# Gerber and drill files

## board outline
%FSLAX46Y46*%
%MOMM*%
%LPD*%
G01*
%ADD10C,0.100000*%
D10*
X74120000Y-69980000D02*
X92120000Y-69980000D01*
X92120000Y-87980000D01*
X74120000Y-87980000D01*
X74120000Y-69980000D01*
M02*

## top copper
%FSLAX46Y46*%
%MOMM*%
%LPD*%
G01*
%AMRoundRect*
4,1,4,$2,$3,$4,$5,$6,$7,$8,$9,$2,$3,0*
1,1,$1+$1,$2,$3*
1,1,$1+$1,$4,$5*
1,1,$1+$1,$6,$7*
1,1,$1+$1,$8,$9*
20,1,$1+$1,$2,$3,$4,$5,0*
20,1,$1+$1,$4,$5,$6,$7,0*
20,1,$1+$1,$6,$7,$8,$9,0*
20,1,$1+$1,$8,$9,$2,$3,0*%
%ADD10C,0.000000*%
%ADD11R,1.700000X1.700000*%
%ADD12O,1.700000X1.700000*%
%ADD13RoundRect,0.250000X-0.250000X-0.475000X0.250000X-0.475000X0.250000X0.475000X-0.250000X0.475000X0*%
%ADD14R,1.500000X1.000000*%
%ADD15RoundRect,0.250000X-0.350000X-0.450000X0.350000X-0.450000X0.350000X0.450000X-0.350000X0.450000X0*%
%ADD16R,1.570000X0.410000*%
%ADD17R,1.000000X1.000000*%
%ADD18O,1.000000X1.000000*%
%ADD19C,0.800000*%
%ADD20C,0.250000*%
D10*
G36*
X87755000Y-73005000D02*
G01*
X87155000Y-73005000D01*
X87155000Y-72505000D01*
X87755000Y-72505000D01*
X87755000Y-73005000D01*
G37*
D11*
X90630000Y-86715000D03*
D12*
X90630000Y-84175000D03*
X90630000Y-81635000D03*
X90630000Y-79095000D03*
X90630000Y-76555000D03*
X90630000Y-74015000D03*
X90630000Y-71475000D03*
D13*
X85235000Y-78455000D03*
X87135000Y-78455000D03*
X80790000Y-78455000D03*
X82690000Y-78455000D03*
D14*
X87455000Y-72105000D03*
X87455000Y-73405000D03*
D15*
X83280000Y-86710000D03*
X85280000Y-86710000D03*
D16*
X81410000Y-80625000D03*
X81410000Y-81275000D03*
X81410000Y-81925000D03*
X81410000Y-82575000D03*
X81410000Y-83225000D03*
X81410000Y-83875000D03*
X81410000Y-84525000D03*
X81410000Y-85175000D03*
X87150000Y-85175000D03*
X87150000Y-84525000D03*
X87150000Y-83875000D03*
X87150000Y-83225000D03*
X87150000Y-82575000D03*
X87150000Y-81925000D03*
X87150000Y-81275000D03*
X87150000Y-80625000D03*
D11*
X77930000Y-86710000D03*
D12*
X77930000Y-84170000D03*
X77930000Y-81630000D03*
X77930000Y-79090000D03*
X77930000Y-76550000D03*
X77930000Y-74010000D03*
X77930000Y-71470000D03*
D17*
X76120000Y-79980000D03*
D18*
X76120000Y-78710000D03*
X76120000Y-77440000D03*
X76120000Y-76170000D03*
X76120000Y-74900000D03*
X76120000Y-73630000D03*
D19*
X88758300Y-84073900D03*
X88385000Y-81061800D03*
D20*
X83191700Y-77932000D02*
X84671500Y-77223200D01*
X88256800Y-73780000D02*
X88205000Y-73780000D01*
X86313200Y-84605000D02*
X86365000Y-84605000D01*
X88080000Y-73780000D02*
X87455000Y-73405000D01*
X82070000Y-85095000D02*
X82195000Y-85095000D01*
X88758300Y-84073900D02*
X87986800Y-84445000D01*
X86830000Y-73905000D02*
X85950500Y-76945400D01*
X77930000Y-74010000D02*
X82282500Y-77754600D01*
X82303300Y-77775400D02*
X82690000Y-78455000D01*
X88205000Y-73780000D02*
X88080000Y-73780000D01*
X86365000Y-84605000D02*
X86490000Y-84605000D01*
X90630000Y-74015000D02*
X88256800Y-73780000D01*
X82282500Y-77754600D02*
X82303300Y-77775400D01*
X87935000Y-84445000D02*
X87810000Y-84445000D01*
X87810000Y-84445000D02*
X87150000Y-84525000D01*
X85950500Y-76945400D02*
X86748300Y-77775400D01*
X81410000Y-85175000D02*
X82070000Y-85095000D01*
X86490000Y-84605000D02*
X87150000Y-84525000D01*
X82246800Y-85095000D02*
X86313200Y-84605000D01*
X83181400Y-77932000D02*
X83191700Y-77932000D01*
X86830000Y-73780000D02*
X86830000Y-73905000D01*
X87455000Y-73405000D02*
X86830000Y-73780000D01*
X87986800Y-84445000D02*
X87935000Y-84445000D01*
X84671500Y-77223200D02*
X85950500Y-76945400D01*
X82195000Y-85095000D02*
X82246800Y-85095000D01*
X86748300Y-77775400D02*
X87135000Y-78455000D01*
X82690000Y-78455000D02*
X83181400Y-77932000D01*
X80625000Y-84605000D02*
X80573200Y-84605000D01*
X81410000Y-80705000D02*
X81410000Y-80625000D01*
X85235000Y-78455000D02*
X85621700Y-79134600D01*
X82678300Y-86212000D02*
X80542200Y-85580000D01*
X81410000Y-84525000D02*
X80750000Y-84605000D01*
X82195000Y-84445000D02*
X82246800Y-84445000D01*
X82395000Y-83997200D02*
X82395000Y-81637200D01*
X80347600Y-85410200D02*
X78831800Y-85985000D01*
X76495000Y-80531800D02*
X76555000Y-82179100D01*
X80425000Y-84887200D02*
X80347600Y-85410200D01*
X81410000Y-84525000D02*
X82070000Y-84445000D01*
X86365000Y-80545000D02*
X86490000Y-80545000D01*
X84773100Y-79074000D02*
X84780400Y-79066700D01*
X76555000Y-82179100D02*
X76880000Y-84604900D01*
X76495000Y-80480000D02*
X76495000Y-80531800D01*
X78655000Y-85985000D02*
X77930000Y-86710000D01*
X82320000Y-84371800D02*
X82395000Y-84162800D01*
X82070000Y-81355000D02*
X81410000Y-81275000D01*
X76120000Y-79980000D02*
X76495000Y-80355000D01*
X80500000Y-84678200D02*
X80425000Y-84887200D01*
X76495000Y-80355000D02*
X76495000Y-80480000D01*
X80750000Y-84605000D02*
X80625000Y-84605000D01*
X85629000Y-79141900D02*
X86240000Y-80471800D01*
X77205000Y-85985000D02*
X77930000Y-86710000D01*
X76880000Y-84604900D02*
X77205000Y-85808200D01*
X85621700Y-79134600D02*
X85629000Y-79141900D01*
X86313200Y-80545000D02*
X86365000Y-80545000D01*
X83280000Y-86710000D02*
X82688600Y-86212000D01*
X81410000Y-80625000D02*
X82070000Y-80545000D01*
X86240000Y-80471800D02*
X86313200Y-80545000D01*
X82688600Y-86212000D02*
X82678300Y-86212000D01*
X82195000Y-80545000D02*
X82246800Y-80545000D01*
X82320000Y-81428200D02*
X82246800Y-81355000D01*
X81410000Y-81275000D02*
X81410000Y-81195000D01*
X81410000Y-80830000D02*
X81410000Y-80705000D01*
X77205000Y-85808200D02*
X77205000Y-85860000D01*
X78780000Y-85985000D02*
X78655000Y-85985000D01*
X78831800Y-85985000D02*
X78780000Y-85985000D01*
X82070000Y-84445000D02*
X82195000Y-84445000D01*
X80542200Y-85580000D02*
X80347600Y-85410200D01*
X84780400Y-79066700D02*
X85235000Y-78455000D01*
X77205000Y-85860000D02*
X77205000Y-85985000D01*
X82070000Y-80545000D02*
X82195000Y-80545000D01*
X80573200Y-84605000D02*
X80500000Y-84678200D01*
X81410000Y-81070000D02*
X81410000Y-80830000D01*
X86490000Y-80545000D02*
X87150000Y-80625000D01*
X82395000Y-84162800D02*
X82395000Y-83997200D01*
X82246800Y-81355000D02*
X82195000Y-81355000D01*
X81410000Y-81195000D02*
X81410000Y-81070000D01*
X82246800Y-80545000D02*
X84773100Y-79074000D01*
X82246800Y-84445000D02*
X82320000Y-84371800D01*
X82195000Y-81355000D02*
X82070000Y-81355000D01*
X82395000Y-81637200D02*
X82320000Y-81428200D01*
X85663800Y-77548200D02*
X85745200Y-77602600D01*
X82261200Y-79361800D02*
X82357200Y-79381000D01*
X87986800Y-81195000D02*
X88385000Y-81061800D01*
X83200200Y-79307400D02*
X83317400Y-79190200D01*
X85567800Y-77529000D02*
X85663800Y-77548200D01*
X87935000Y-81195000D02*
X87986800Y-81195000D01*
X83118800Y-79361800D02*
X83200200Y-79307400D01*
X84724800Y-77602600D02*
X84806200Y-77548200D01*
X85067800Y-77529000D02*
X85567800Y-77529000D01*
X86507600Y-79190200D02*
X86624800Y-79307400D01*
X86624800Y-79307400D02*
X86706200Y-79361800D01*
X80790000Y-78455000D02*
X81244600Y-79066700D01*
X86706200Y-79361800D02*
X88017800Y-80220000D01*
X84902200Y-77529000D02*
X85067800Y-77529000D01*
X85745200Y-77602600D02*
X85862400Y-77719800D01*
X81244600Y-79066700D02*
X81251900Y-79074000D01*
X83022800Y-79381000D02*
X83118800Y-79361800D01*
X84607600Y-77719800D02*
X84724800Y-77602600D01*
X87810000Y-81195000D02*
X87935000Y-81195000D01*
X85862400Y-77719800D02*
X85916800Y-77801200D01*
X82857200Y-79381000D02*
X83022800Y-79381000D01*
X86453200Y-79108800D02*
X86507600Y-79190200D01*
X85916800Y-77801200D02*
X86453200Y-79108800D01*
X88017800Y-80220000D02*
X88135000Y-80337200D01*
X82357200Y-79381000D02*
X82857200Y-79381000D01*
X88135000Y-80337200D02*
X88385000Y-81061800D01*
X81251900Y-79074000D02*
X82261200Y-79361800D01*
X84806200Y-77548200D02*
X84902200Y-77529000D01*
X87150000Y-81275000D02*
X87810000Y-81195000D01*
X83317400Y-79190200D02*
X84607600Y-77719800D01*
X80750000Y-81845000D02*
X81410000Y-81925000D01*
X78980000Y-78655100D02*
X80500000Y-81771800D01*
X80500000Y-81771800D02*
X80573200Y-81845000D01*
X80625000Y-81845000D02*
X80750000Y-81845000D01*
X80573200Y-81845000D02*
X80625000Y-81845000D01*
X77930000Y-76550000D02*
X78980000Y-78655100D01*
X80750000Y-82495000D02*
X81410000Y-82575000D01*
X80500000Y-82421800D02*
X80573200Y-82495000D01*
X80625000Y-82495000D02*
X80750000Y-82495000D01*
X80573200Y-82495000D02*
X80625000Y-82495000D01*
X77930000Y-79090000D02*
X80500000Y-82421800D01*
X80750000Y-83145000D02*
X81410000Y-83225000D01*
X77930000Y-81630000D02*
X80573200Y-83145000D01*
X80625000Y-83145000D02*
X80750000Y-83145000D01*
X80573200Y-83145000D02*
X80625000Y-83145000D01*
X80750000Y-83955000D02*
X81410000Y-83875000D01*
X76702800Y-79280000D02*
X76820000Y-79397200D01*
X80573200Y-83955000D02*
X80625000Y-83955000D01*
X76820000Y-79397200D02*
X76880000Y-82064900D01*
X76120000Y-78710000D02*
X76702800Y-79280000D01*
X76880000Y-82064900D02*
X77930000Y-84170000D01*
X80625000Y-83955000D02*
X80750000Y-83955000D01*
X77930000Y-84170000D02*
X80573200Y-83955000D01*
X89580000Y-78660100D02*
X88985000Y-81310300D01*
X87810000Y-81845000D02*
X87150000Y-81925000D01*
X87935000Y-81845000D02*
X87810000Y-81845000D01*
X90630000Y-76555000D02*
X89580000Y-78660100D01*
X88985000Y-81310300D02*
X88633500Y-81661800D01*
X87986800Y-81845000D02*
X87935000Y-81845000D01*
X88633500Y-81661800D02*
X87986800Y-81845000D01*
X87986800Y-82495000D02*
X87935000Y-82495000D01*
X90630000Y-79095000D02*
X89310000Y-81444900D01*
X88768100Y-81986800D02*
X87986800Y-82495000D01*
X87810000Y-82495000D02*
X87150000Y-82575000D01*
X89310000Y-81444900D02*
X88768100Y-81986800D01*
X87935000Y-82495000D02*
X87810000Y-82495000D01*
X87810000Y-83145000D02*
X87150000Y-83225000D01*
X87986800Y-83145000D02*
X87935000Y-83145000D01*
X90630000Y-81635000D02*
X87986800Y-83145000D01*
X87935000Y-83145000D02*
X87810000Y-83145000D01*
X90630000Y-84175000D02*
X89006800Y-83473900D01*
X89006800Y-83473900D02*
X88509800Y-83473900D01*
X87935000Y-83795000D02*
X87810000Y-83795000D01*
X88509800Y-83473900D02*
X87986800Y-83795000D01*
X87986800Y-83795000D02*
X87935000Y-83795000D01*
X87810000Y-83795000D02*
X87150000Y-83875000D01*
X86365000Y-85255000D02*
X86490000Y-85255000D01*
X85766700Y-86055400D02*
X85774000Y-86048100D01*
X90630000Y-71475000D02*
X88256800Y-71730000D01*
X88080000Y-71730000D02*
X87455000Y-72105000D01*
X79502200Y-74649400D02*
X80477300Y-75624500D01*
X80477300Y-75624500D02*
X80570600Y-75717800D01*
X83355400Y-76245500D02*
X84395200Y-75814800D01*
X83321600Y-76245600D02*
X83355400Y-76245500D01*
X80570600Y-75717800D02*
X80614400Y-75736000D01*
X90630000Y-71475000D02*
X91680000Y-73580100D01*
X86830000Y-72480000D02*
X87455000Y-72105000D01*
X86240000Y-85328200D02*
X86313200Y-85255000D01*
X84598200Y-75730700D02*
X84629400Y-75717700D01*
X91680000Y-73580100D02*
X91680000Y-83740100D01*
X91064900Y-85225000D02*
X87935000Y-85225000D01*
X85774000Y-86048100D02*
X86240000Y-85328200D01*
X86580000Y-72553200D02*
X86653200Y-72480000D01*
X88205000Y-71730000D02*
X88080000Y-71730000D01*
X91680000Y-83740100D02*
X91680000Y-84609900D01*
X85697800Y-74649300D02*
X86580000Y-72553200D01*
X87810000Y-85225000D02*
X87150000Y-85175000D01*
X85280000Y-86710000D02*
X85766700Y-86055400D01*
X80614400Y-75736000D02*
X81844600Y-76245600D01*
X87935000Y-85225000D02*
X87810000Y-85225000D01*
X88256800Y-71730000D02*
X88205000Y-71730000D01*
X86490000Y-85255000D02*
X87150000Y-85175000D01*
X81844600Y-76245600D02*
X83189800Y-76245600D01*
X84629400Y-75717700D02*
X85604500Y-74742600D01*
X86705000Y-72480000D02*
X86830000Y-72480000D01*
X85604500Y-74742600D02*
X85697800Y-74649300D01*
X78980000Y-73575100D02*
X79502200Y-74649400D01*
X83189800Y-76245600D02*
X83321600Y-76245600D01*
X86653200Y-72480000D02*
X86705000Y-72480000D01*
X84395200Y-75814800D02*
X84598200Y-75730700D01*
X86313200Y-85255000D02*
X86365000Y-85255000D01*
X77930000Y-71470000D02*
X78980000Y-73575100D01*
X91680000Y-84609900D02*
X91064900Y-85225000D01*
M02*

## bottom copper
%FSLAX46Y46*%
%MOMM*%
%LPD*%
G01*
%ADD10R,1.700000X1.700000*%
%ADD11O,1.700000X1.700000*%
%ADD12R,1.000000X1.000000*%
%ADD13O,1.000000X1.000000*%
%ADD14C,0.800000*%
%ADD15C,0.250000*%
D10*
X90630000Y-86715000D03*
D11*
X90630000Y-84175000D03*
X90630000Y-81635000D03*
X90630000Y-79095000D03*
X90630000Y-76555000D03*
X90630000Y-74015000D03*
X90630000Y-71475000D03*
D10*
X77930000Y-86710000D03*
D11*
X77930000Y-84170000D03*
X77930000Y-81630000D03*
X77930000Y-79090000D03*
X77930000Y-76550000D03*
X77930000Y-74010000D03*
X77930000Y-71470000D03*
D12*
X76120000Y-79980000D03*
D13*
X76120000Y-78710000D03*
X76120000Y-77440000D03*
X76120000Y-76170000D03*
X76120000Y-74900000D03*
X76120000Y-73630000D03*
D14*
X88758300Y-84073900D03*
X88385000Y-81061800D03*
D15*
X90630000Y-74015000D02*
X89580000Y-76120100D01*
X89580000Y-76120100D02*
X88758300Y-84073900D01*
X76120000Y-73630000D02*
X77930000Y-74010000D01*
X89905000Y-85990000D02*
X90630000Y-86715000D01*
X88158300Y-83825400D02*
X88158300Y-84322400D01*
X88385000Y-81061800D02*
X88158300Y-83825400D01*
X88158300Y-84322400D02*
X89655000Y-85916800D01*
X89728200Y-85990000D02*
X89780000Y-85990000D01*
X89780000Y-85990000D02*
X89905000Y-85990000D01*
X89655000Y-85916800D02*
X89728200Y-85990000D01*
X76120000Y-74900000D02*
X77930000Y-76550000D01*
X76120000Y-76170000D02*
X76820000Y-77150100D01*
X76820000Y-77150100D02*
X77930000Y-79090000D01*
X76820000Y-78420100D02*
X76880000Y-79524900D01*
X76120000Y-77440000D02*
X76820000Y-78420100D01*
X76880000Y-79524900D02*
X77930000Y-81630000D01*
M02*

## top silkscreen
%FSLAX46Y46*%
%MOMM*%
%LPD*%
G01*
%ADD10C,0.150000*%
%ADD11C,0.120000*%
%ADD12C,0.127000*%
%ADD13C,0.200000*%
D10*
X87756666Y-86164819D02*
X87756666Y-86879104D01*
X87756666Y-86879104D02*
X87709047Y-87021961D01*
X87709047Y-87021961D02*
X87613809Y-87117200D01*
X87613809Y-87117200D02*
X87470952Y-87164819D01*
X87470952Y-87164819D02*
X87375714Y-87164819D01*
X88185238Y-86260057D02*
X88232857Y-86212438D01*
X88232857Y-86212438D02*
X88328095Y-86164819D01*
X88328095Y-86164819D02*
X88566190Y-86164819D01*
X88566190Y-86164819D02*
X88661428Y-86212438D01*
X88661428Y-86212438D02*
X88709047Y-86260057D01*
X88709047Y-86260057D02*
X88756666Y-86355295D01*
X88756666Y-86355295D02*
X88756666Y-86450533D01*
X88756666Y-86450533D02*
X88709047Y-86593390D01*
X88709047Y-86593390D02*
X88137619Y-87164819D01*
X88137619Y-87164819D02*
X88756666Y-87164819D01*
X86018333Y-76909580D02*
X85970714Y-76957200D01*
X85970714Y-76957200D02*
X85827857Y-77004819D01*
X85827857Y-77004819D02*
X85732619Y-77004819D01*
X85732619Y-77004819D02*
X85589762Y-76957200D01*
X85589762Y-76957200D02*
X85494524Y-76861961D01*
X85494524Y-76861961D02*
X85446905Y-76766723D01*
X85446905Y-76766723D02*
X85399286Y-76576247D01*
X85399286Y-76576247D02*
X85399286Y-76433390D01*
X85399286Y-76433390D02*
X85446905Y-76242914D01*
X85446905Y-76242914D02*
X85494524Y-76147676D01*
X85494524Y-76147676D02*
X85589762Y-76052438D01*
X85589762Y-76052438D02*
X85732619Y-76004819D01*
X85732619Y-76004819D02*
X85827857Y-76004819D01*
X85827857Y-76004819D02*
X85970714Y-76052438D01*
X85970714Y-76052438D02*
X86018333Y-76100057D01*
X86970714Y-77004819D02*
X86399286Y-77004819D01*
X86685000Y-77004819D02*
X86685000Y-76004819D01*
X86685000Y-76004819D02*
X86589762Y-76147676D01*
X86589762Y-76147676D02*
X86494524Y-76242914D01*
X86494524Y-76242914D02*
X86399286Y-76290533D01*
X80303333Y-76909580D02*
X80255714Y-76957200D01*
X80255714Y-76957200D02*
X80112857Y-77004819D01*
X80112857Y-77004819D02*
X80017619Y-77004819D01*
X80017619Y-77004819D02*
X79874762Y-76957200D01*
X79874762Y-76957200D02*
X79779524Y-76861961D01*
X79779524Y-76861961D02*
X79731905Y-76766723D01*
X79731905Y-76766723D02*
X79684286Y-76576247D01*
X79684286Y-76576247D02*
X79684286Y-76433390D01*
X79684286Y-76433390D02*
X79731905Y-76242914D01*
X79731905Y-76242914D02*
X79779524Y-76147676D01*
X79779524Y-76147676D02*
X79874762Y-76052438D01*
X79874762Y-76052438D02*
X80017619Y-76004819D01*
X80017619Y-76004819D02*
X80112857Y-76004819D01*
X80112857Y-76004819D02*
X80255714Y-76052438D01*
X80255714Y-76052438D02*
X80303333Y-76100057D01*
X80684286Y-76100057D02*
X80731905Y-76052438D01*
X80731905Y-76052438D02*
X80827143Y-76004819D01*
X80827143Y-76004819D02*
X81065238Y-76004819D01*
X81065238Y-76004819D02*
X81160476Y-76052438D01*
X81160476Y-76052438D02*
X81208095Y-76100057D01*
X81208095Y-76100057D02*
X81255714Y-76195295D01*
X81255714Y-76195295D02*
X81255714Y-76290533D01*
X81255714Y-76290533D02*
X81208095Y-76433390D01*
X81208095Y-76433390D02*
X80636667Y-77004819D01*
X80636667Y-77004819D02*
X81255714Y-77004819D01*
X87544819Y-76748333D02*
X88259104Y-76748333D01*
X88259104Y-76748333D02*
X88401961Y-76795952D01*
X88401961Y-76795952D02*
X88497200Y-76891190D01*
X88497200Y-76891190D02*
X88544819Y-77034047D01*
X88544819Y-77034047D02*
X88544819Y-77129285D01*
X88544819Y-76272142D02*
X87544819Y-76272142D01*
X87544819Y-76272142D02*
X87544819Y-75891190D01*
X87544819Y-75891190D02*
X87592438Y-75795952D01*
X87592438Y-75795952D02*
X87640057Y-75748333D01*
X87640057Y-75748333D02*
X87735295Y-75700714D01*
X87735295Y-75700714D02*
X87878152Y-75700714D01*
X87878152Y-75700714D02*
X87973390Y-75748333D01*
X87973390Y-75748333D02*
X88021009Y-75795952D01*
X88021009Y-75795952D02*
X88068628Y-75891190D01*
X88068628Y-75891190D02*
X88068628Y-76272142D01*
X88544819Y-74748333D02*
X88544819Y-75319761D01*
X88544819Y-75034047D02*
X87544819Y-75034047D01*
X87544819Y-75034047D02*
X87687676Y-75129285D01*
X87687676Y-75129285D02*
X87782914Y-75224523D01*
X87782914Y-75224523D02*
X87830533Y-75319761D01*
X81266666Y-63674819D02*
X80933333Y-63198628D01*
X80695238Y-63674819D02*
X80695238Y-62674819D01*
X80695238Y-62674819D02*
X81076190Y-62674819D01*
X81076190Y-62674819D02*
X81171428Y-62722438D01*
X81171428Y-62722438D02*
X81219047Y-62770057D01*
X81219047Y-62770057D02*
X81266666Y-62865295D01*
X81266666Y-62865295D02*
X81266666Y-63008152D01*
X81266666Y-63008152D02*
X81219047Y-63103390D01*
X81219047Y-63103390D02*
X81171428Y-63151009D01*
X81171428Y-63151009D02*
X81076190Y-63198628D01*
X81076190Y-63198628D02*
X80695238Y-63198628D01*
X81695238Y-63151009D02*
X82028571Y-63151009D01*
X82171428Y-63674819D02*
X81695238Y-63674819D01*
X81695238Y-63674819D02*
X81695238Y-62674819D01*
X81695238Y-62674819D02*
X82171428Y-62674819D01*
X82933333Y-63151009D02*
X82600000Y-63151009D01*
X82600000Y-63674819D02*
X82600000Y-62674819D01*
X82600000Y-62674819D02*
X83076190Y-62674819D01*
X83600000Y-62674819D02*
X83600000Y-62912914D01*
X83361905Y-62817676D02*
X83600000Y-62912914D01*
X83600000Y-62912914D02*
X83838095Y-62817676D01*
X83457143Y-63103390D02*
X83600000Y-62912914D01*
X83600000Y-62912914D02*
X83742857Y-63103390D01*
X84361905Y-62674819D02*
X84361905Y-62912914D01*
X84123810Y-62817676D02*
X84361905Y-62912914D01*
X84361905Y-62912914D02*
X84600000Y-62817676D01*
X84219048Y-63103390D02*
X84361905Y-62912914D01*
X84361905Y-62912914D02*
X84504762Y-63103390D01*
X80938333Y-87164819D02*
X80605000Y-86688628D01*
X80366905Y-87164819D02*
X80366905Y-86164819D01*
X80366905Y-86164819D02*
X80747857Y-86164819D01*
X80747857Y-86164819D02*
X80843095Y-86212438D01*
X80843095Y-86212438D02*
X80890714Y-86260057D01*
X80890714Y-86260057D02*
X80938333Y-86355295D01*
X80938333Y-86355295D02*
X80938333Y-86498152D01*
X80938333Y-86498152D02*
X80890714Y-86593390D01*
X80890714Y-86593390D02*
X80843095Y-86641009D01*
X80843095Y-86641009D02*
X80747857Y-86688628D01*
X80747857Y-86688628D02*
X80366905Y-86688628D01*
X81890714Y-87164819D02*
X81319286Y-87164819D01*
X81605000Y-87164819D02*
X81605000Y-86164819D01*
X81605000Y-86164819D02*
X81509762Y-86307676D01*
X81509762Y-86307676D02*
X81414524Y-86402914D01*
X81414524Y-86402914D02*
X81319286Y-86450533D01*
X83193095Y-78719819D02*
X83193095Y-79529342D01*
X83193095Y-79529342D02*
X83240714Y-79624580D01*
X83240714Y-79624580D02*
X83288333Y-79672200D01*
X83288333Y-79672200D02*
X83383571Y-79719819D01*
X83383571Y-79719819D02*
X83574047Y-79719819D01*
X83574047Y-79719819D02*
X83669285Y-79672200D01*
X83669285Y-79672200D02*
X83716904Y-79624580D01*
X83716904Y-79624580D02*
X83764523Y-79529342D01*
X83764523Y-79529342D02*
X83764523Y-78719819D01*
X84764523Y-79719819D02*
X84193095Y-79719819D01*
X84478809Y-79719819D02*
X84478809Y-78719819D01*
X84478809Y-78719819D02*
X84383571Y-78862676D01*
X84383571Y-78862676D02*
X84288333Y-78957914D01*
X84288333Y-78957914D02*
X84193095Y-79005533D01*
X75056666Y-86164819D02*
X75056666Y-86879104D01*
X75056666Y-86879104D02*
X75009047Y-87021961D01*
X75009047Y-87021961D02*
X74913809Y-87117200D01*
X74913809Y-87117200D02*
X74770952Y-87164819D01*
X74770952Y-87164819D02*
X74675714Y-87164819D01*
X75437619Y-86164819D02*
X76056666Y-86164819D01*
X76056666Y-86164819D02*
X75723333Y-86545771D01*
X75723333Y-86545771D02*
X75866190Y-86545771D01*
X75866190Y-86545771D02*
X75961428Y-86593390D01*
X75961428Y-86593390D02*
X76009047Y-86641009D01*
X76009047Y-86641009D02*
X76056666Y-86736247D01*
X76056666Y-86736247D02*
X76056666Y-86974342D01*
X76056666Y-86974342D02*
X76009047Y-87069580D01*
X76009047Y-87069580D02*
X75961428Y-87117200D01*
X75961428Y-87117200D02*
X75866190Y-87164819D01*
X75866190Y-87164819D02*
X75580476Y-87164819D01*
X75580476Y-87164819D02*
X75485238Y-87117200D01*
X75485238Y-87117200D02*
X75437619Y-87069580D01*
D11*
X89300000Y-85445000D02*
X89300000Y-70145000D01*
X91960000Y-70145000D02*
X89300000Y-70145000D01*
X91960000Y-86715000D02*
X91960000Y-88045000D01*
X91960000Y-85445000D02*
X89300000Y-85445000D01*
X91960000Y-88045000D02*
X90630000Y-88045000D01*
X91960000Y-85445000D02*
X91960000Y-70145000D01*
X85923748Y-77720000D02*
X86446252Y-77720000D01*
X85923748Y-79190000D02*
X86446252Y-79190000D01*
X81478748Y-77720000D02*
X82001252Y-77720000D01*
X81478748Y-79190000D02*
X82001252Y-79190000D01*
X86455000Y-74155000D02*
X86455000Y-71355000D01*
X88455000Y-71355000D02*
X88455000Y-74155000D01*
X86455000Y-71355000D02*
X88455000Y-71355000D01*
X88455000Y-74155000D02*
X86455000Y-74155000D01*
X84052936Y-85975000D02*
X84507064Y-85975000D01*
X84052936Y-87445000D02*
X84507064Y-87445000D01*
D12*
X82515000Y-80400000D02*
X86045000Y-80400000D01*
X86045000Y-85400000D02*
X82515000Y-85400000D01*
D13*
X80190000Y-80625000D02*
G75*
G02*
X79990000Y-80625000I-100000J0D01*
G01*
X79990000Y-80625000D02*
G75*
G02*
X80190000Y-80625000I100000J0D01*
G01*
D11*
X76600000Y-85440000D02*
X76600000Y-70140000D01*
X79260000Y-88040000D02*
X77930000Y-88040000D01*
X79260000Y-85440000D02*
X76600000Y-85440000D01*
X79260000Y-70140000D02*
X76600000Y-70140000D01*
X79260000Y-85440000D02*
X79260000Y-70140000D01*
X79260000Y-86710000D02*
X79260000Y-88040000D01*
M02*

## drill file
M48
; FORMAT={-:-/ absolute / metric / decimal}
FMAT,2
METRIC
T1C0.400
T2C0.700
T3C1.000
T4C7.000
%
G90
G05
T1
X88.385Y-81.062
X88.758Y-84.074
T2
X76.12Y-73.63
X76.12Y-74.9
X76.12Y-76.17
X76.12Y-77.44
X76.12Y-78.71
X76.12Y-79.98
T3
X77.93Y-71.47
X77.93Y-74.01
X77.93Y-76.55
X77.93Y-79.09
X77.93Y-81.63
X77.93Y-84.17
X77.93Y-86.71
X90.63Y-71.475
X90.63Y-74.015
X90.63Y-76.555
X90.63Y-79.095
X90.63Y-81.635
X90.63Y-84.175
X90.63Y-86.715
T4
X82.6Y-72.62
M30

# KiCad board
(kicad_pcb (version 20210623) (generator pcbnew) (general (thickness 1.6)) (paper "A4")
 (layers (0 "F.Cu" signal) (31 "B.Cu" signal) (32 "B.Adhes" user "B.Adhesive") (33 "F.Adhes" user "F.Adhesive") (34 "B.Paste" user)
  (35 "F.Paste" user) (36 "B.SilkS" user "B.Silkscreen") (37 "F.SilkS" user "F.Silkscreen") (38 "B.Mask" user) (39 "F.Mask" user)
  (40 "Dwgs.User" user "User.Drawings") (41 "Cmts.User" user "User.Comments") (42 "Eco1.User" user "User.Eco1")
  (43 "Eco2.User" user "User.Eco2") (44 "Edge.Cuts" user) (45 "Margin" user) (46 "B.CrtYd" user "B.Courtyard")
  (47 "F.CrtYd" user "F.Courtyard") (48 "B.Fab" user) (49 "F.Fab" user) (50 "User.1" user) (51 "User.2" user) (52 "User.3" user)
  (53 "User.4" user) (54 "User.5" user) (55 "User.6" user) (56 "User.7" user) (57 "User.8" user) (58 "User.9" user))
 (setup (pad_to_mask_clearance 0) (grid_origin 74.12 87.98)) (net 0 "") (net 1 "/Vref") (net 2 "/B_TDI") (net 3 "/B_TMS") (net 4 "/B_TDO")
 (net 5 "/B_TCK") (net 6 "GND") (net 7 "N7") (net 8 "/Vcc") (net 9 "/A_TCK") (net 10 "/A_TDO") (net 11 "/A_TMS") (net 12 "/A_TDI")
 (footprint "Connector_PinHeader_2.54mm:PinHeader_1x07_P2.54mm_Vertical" (layer "F.Cu") (at 90.63 86.715 180)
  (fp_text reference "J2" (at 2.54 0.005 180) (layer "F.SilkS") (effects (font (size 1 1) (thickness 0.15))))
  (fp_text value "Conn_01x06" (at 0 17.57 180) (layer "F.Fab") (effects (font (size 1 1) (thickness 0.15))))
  (fp_line (start 1.33 1.27) (end 1.33 16.57) (layer "F.SilkS") (width 0.12))
  (fp_line (start -1.33 16.57) (end 1.33 16.57) (layer "F.SilkS") (width 0.12))
  (fp_line (start -1.33 0) (end -1.33 -1.33) (layer "F.SilkS") (width 0.12))
  (fp_line (start -1.33 1.27) (end 1.33 1.27) (layer "F.SilkS") (width 0.12))
  (fp_line (start -1.33 -1.33) (end 0 -1.33) (layer "F.SilkS") (width 0.12))
  (fp_line (start -1.33 1.27) (end -1.33 16.57) (layer "F.SilkS") (width 0.12))
  (pad "1" thru_hole rect locked (at 0 0 180) (size 1.7 1.7) (drill 1) (layers *.Cu *.Mask) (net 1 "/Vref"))
  (pad "2" thru_hole oval locked (at 0 2.54 180) (size 1.7 1.7) (drill 1) (layers *.Cu *.Mask) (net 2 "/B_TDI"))
  (pad "3" thru_hole oval locked (at 0 5.08 180) (size 1.7 1.7) (drill 1) (layers *.Cu *.Mask) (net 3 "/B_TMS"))
  (pad "4" thru_hole oval locked (at 0 7.62 180) (size 1.7 1.7) (drill 1) (layers *.Cu *.Mask) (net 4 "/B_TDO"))
  (pad "5" thru_hole oval locked (at 0 10.16 180) (size 1.7 1.7) (drill 1) (layers *.Cu *.Mask) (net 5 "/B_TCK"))
  (pad "6" thru_hole oval locked (at 0 12.7 180) (size 1.7 1.7) (drill 1) (layers *.Cu *.Mask) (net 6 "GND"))
  (pad "7" thru_hole oval locked (at 0 15.24 180) (size 1.7 1.7) (drill 1) (layers *.Cu *.Mask) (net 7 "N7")))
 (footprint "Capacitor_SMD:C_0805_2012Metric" (layer "F.Cu") (at 86.185 78.455)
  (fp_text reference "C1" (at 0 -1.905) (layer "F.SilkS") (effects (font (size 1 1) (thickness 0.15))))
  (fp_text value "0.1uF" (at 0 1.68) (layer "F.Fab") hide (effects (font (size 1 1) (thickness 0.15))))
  (fp_line (start -0.261252 -0.735) (end 0.261252 -0.735) (layer "F.SilkS") (width 0.12))
  (fp_line (start -0.261252 0.735) (end 0.261252 0.735) (layer "F.SilkS") (width 0.12))
  (pad "1" smd roundrect locked (at -0.95 0) (size 1 1.45) (layers "F.Cu" "F.Paste" "F.Mask") (roundrect_rratio 0.25) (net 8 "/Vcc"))
  (pad "2" smd roundrect locked (at 0.95 0) (size 1 1.45) (layers "F.Cu" "F.Paste" "F.Mask") (roundrect_rratio 0.25) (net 6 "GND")))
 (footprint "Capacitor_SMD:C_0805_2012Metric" (layer "F.Cu") (at 81.74 78.455)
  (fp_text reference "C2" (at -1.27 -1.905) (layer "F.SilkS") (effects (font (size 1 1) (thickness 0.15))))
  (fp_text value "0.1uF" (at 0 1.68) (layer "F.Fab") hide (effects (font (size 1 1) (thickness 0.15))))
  (fp_line (start -0.261252 -0.735) (end 0.261252 -0.735) (layer "F.SilkS") (width 0.12))
  (fp_line (start -0.261252 0.735) (end 0.261252 0.735) (layer "F.SilkS") (width 0.12))
  (pad "1" smd roundrect locked (at -0.95 0) (size 1 1.45) (layers "F.Cu" "F.Paste" "F.Mask") (roundrect_rratio 0.25) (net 1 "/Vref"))
  (pad "2" smd roundrect locked (at 0.95 0) (size 1 1.45) (layers "F.Cu" "F.Paste" "F.Mask") (roundrect_rratio 0.25) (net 6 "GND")))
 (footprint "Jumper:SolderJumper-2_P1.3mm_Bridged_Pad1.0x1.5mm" (layer "F.Cu") (at 87.455 72.755 -90)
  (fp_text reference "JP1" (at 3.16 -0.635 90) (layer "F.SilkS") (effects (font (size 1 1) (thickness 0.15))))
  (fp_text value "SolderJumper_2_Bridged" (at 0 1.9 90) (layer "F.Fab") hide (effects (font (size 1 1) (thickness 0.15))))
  (fp_poly (pts (xy -0.25 -0.3) (xy 0.25 -0.3) (xy 0.25 0.3) (xy -0.25 0.3)) (layer "F.Cu") (width 0) (fill solid))
  (fp_line (start 1.4 1) (end -1.4 1) (layer "F.SilkS") (width 0.12))
  (fp_line (start -1.4 -1) (end 1.4 -1) (layer "F.SilkS") (width 0.12))
  (fp_line (start -1.4 1) (end -1.4 -1) (layer "F.SilkS") (width 0.12))
  (fp_line (start 1.4 -1) (end 1.4 1) (layer "F.SilkS") (width 0.12))
  (pad "1" smd rect locked (at -0.65 0 270) (size 1 1.5) (layers "F.Cu" "F.Mask") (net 7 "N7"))
  (pad "2" smd rect locked (at 0.65 0 270) (size 1 1.5) (layers "F.Cu" "F.Mask") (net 6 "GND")))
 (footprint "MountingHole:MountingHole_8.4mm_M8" (layer "F.Cu") (at 82.6 72.62)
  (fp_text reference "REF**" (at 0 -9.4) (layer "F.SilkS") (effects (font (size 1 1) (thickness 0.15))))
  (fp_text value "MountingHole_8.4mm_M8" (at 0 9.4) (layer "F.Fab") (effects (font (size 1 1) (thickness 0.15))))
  (pad "" np_thru_hole circle (at 0 0) (size 7 7) (drill 7) (layers F&B.Cu *.Mask)))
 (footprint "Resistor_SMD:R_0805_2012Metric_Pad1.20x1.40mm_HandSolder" (layer "F.Cu") (at 84.28 86.71)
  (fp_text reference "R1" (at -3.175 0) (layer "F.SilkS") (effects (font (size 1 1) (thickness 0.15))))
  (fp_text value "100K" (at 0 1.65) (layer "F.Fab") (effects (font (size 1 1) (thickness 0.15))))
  (fp_line (start -0.227064 -0.735) (end 0.227064 -0.735) (layer "F.SilkS") (width 0.12))
  (fp_line (start -0.227064 0.735) (end 0.227064 0.735) (layer "F.SilkS") (width 0.12))
  (pad "1" smd roundrect locked (at -1 0) (size 1.2 1.4) (layers "F.Cu" "F.Paste" "F.Mask") (roundrect_rratio 0.208333) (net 8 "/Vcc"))
  (pad "2" smd roundrect locked (at 1 0) (size 1.2 1.4) (layers "F.Cu" "F.Paste" "F.Mask") (roundrect_rratio 0.208333) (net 7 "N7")))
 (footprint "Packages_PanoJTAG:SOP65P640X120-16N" (layer "F.Cu") (at 84.28 82.9)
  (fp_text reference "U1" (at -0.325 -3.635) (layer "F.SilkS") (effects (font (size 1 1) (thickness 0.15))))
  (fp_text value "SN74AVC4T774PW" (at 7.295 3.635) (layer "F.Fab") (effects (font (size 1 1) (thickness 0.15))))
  (fp_line (start -1.765 -2.5) (end 1.765 -2.5) (layer "F.SilkS") (width 0.127))
  (fp_line (start 1.765 2.5) (end -1.765 2.5) (layer "F.SilkS") (width 0.127))
  (fp_circle (center -4.19 -2.275) (end -4.09 -2.275) (layer "F.SilkS") (width 0.2) (fill none))
  (pad "1" smd rect locked (at -2.87 -2.275) (size 1.57 0.41) (layers "F.Cu" "F.Paste" "F.Mask") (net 8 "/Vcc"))
  (pad "2" smd rect locked (at -2.87 -1.625) (size 1.57 0.41) (layers "F.Cu" "F.Paste" "F.Mask") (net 8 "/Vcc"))
  (pad "3" smd rect locked (at -2.87 -0.975) (size 1.57 0.41) (layers "F.Cu" "F.Paste" "F.Mask") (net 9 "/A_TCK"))
  (pad "4" smd rect locked (at -2.87 -0.325) (size 1.57 0.41) (layers "F.Cu" "F.Paste" "F.Mask") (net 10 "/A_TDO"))
  (pad "5" smd rect locked (at -2.87 0.325) (size 1.57 0.41) (layers "F.Cu" "F.Paste" "F.Mask") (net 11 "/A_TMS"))
  (pad "6" smd rect locked (at -2.87 0.975) (size 1.57 0.41) (layers "F.Cu" "F.Paste" "F.Mask") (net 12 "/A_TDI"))
  (pad "7" smd rect locked (at -2.87 1.625) (size 1.57 0.41) (layers "F.Cu" "F.Paste" "F.Mask") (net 8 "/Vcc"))
  (pad "8" smd rect locked (at -2.87 2.275) (size 1.57 0.41) (layers "F.Cu" "F.Paste" "F.Mask") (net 6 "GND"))
  (pad "9" smd rect locked (at 2.87 2.275) (size 1.57 0.41) (layers "F.Cu" "F.Paste" "F.Mask") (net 7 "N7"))
  (pad "10" smd rect locked (at 2.87 1.625) (size 1.57 0.41) (layers "F.Cu" "F.Paste" "F.Mask") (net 6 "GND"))
  (pad "11" smd rect locked (at 2.87 0.975) (size 1.57 0.41) (layers "F.Cu" "F.Paste" "F.Mask") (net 2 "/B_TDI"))
  (pad "12" smd rect locked (at 2.87 0.325) (size 1.57 0.41) (layers "F.Cu" "F.Paste" "F.Mask") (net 3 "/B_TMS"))
  (pad "13" smd rect locked (at 2.87 -0.325) (size 1.57 0.41) (layers "F.Cu" "F.Paste" "F.Mask") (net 4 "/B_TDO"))
  (pad "14" smd rect locked (at 2.87 -0.975) (size 1.57 0.41) (layers "F.Cu" "F.Paste" "F.Mask") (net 5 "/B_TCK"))
  (pad "15" smd rect locked (at 2.87 -1.625) (size 1.57 0.41) (layers "F.Cu" "F.Paste" "F.Mask") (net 1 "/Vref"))
  (pad "16" smd rect locked (at 2.87 -2.275) (size 1.57 0.41) (layers "F.Cu" "F.Paste" "F.Mask") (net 8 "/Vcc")))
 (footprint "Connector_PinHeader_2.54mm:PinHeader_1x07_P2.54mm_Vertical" (layer "F.Cu") (at 77.93 86.71 180)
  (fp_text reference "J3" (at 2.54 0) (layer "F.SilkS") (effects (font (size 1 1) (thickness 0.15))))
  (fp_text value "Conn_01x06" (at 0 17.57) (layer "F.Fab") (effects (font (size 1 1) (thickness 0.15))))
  (fp_line (start 1.33 1.27) (end 1.33 16.57) (layer "F.SilkS") (width 0.12))
  (fp_line (start -1.33 -1.33) (end 0 -1.33) (layer "F.SilkS") (width 0.12))
  (fp_line (start -1.33 1.27) (end 1.33 1.27) (layer "F.SilkS") (width 0.12))
  (fp_line (start -1.33 16.57) (end 1.33 16.57) (layer "F.SilkS") (width 0.12))
  (fp_line (start -1.33 1.27) (end -1.33 16.57) (layer "F.SilkS") (width 0.12))
  (fp_line (start -1.33 0) (end -1.33 -1.33) (layer "F.SilkS") (width 0.12))
  (pad "1" thru_hole rect locked (at 0 0 180) (size 1.7 1.7) (drill 1) (layers *.Cu *.Mask) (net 8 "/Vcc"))
  (pad "2" thru_hole oval locked (at 0 2.54 180) (size 1.7 1.7) (drill 1) (layers *.Cu *.Mask) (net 12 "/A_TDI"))
  (pad "3" thru_hole oval locked (at 0 5.08 180) (size 1.7 1.7) (drill 1) (layers *.Cu *.Mask) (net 11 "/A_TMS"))
  (pad "4" thru_hole oval locked (at 0 7.62 180) (size 1.7 1.7) (drill 1) (layers *.Cu *.Mask) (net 10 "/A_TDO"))
  (pad "5" thru_hole oval locked (at 0 10.16 180) (size 1.7 1.7) (drill 1) (layers *.Cu *.Mask) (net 9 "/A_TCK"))
  (pad "6" thru_hole oval locked (at 0 12.7 180) (size 1.7 1.7) (drill 1) (layers *.Cu *.Mask) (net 6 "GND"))
  (pad "7" thru_hole oval locked (at 0 15.24 180) (size 1.7 1.7) (drill 1) (layers *.Cu *.Mask) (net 7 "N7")))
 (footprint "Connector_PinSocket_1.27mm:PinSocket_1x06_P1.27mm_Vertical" (layer "B.Cu") (at 76.12 79.98)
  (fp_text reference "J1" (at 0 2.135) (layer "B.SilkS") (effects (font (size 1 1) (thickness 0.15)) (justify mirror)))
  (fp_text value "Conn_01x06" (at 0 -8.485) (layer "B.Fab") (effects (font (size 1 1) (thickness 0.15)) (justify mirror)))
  (pad "1" thru_hole rect locked (at 0 0) (size 1 1) (drill 0.7) (layers *.Cu *.Mask) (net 8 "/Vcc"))
  (pad "2" thru_hole oval locked (at 0 -1.27) (size 1 1) (drill 0.7) (layers *.Cu *.Mask) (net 12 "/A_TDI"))
  (pad "3" thru_hole oval locked (at 0 -2.54) (size 1 1) (drill 0.7) (layers *.Cu *.Mask) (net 11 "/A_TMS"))
  (pad "4" thru_hole oval locked (at 0 -3.81) (size 1 1) (drill 0.7) (layers *.Cu *.Mask) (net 10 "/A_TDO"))
  (pad "5" thru_hole oval locked (at 0 -5.08) (size 1 1) (drill 0.7) (layers *.Cu *.Mask) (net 9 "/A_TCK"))
  (pad "6" thru_hole oval locked (at 0 -6.35) (size 1 1) (drill 0.7) (layers *.Cu *.Mask) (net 6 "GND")))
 (gr_rect (start 92.12 87.98) (end 74.12 69.98) (layer "Edge.Cuts") (width 0.1) (fill none))
 (segment (start 83.1917 77.932) (end 84.6715 77.2232) (width 0.25) (layer "F.Cu") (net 6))
 (segment (start 88.2568 73.78) (end 88.205 73.78) (width 0.25) (layer "F.Cu") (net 6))
 (segment (start 86.3132 84.605) (end 86.365 84.605) (width 0.25) (layer "F.Cu") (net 6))
 (segment (start 88.08 73.78) (end 87.455 73.405) (width 0.25) (layer "F.Cu") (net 6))
 (segment (start 82.07 85.095) (end 82.195 85.095) (width 0.25) (layer "F.Cu") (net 6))
 (segment (start 88.7583 84.0739) (end 87.9868 84.445) (width 0.25) (layer "F.Cu") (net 6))
 (segment (start 86.83 73.905) (end 85.9505 76.9454) (width 0.25) (layer "F.Cu") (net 6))
 (segment (start 77.93 74.01) (end 82.2825 77.7546) (width 0.25) (layer "F.Cu") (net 6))
 (segment (start 82.3033 77.7754) (end 82.69 78.455) (width 0.25) (layer "F.Cu") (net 6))
 (segment (start 88.205 73.78) (end 88.08 73.78) (width 0.25) (layer "F.Cu") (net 6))
 (segment (start 86.365 84.605) (end 86.49 84.605) (width 0.25) (layer "F.Cu") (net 6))
 (segment (start 90.63 74.015) (end 88.2568 73.78) (width 0.25) (layer "F.Cu") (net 6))
 (segment (start 82.2825 77.7546) (end 82.3033 77.7754) (width 0.25) (layer "F.Cu") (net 6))
 (segment (start 87.935 84.445) (end 87.81 84.445) (width 0.25) (layer "F.Cu") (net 6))
 (segment (start 87.81 84.445) (end 87.15 84.525) (width 0.25) (layer "F.Cu") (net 6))
 (segment (start 85.9505 76.9454) (end 86.7483 77.7754) (width 0.25) (layer "F.Cu") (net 6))
 (segment (start 81.41 85.175) (end 82.07 85.095) (width 0.25) (layer "F.Cu") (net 6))
 (segment (start 86.49 84.605) (end 87.15 84.525) (width 0.25) (layer "F.Cu") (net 6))
 (segment (start 82.2468 85.095) (end 86.3132 84.605) (width 0.25) (layer "F.Cu") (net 6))
 (segment (start 83.1814 77.932) (end 83.1917 77.932) (width 0.25) (layer "F.Cu") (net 6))
 (segment (start 86.83 73.78) (end 86.83 73.905) (width 0.25) (layer "F.Cu") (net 6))
 (segment (start 87.455 73.405) (end 86.83 73.78) (width 0.25) (layer "F.Cu") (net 6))
 (segment (start 87.9868 84.445) (end 87.935 84.445) (width 0.25) (layer "F.Cu") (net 6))
 (segment (start 84.6715 77.2232) (end 85.9505 76.9454) (width 0.25) (layer "F.Cu") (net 6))
 (segment (start 82.195 85.095) (end 82.2468 85.095) (width 0.25) (layer "F.Cu") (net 6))
 (segment (start 86.7483 77.7754) (end 87.135 78.455) (width 0.25) (layer "F.Cu") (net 6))
 (segment (start 82.69 78.455) (end 83.1814 77.932) (width 0.25) (layer "F.Cu") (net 6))
 (via (at 88.7583 84.0739) (size 0.8) (drill 0.4) (layers "F.Cu" "B.Cu") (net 6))
 (segment (start 90.63 74.015) (end 89.58 76.1201) (width 0.25) (layer "B.Cu") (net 6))
 (segment (start 89.58 76.1201) (end 88.7583 84.0739) (width 0.25) (layer "B.Cu") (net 6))
 (segment (start 76.12 73.63) (end 77.93 74.01) (width 0.25) (layer "B.Cu") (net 6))
 (segment (start 80.625 84.605) (end 80.5732 84.605) (width 0.25) (layer "F.Cu") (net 8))
 (segment (start 81.41 80.705) (end 81.41 80.625) (width 0.25) (layer "F.Cu") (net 8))
 (segment (start 85.235 78.455) (end 85.6217 79.1346) (width 0.25) (layer "F.Cu") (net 8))
 (segment (start 82.6783 86.212) (end 80.5422 85.58) (width 0.25) (layer "F.Cu") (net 8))
 (segment (start 81.41 84.525) (end 80.75 84.605) (width 0.25) (layer "F.Cu") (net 8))
 (segment (start 82.195 84.445) (end 82.2468 84.445) (width 0.25) (layer "F.Cu") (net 8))
 (segment (start 82.395 83.9972) (end 82.395 81.6372) (width 0.25) (layer "F.Cu") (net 8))
 (segment (start 80.3476 85.4102) (end 78.8318 85.985) (width 0.25) (layer "F.Cu") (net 8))
 (segment (start 76.495 80.5318) (end 76.555 82.1791) (width 0.25) (layer "F.Cu") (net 8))
 (segment (start 80.425 84.8872) (end 80.3476 85.4102) (width 0.25) (layer "F.Cu") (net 8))
 (segment (start 81.41 84.525) (end 82.07 84.445) (width 0.25) (layer "F.Cu") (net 8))
 (segment (start 86.365 80.545) (end 86.49 80.545) (width 0.25) (layer "F.Cu") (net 8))
 (segment (start 84.7731 79.074) (end 84.7804 79.0667) (width 0.25) (layer "F.Cu") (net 8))
 (segment (start 76.555 82.1791) (end 76.88 84.6049) (width 0.25) (layer "F.Cu") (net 8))
 (segment (start 76.495 80.48) (end 76.495 80.5318) (width 0.25) (layer "F.Cu") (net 8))
 (segment (start 78.655 85.985) (end 77.93 86.71) (width 0.25) (layer "F.Cu") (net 8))
 (segment (start 82.32 84.3718) (end 82.395 84.1628) (width 0.25) (layer "F.Cu") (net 8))
 (segment (start 82.07 81.355) (end 81.41 81.275) (width 0.25) (layer "F.Cu") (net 8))
 (segment (start 76.12 79.98) (end 76.495 80.355) (width 0.25) (layer "F.Cu") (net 8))
 (segment (start 80.5 84.6782) (end 80.425 84.8872) (width 0.25) (layer "F.Cu") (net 8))
 (segment (start 76.495 80.355) (end 76.495 80.48) (width 0.25) (layer "F.Cu") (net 8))
 (segment (start 80.75 84.605) (end 80.625 84.605) (width 0.25) (layer "F.Cu") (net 8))
 (segment (start 85.629 79.1419) (end 86.24 80.4718) (width 0.25) (layer "F.Cu") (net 8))
 (segment (start 77.205 85.985) (end 77.93 86.71) (width 0.25) (layer "F.Cu") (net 8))
 (segment (start 76.88 84.6049) (end 77.205 85.8082) (width 0.25) (layer "F.Cu") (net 8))
 (segment (start 85.6217 79.1346) (end 85.629 79.1419) (width 0.25) (layer "F.Cu") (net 8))
 (segment (start 86.3132 80.545) (end 86.365 80.545) (width 0.25) (layer "F.Cu") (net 8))
 (segment (start 83.28 86.71) (end 82.6886 86.212) (width 0.25) (layer "F.Cu") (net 8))
 (segment (start 81.41 80.625) (end 82.07 80.545) (width 0.25) (layer "F.Cu") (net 8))
 (segment (start 86.24 80.4718) (end 86.3132 80.545) (width 0.25) (layer "F.Cu") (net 8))
 (segment (start 82.6886 86.212) (end 82.6783 86.212) (width 0.25) (layer "F.Cu") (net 8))
 (segment (start 82.195 80.545) (end 82.2468 80.545) (width 0.25) (layer "F.Cu") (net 8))
 (segment (start 82.32 81.4282) (end 82.2468 81.355) (width 0.25) (layer "F.Cu") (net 8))
 (segment (start 81.41 81.275) (end 81.41 81.195) (width 0.25) (layer "F.Cu") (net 8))
 (segment (start 81.41 80.83) (end 81.41 80.705) (width 0.25) (layer "F.Cu") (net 8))
 (segment (start 77.205 85.8082) (end 77.205 85.86) (width 0.25) (layer "F.Cu") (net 8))
 (segment (start 78.78 85.985) (end 78.655 85.985) (width 0.25) (layer "F.Cu") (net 8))
 (segment (start 78.8318 85.985) (end 78.78 85.985) (width 0.25) (layer "F.Cu") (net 8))
 (segment (start 82.07 84.445) (end 82.195 84.445) (width 0.25) (layer "F.Cu") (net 8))
 (segment (start 80.5422 85.58) (end 80.3476 85.4102) (width 0.25) (layer "F.Cu") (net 8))
 (segment (start 84.7804 79.0667) (end 85.235 78.455) (width 0.25) (layer "F.Cu") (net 8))
 (segment (start 77.205 85.86) (end 77.205 85.985) (width 0.25) (layer "F.Cu") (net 8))
 (segment (start 82.07 80.545) (end 82.195 80.545) (width 0.25) (layer "F.Cu") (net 8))
 (segment (start 80.5732 84.605) (end 80.5 84.6782) (width 0.25) (layer "F.Cu") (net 8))
 (segment (start 81.41 81.07) (end 81.41 80.83) (width 0.25) (layer "F.Cu") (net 8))
 (segment (start 86.49 80.545) (end 87.15 80.625) (width 0.25) (layer "F.Cu") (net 8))
 (segment (start 82.395 84.1628) (end 82.395 83.9972) (width 0.25) (layer "F.Cu") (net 8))
 (segment (start 82.2468 81.355) (end 82.195 81.355) (width 0.25) (layer "F.Cu") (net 8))
 (segment (start 81.41 81.195) (end 81.41 81.07) (width 0.25) (layer "F.Cu") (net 8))
 (segment (start 82.2468 80.545) (end 84.7731 79.074) (width 0.25) (layer "F.Cu") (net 8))
 (segment (start 82.2468 84.445) (end 82.32 84.3718) (width 0.25) (layer "F.Cu") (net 8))
 (segment (start 82.195 81.355) (end 82.07 81.355) (width 0.25) (layer "F.Cu") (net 8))
 (segment (start 82.395 81.6372) (end 82.32 81.4282) (width 0.25) (layer "F.Cu") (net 8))
 (segment (start 85.6638 77.5482) (end 85.7452 77.6026) (width 0.25) (layer "F.Cu") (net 1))
 (segment (start 82.2612 79.3618) (end 82.3572 79.381) (width 0.25) (layer "F.Cu") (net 1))
 (segment (start 87.9868 81.195) (end 88.385 81.0618) (width 0.25) (layer "F.Cu") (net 1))
 (segment (start 83.2002 79.3074) (end 83.3174 79.1902) (width 0.25) (layer "F.Cu") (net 1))
 (segment (start 85.5678 77.529) (end 85.6638 77.5482) (width 0.25) (layer "F.Cu") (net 1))
 (segment (start 87.935 81.195) (end 87.9868 81.195) (width 0.25) (layer "F.Cu") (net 1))
 (segment (start 83.1188 79.3618) (end 83.2002 79.3074) (width 0.25) (layer "F.Cu") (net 1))
 (segment (start 84.7248 77.6026) (end 84.8062 77.5482) (width 0.25) (layer "F.Cu") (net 1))
 (segment (start 85.0678 77.529) (end 85.5678 77.529) (width 0.25) (layer "F.Cu") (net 1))
 (segment (start 86.5076 79.1902) (end 86.6248 79.3074) (width 0.25) (layer "F.Cu") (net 1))
 (segment (start 86.6248 79.3074) (end 86.7062 79.3618) (width 0.25) (layer "F.Cu") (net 1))
 (segment (start 80.79 78.455) (end 81.2446 79.0667) (width 0.25) (layer "F.Cu") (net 1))
 (segment (start 86.7062 79.3618) (end 88.0178 80.22) (width 0.25) (layer "F.Cu") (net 1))
 (segment (start 84.9022 77.529) (end 85.0678 77.529) (width 0.25) (layer "F.Cu") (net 1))
 (segment (start 85.7452 77.6026) (end 85.8624 77.7198) (width 0.25) (layer "F.Cu") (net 1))
 (segment (start 81.2446 79.0667) (end 81.2519 79.074) (width 0.25) (layer "F.Cu") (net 1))
 (segment (start 83.0228 79.381) (end 83.1188 79.3618) (width 0.25) (layer "F.Cu") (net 1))
 (segment (start 84.6076 77.7198) (end 84.7248 77.6026) (width 0.25) (layer "F.Cu") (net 1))
 (segment (start 87.81 81.195) (end 87.935 81.195) (width 0.25) (layer "F.Cu") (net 1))
 (segment (start 85.8624 77.7198) (end 85.9168 77.8012) (width 0.25) (layer "F.Cu") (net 1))
 (segment (start 82.8572 79.381) (end 83.0228 79.381) (width 0.25) (layer "F.Cu") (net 1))
 (segment (start 86.4532 79.1088) (end 86.5076 79.1902) (width 0.25) (layer "F.Cu") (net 1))
 (segment (start 85.9168 77.8012) (end 86.4532 79.1088) (width 0.25) (layer "F.Cu") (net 1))
 (segment (start 88.0178 80.22) (end 88.135 80.3372) (width 0.25) (layer "F.Cu") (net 1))
 (segment (start 82.3572 79.381) (end 82.8572 79.381) (width 0.25) (layer "F.Cu") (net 1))
 (segment (start 88.135 80.3372) (end 88.385 81.0618) (width 0.25) (layer "F.Cu") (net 1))
 (segment (start 81.2519 79.074) (end 82.2612 79.3618) (width 0.25) (layer "F.Cu") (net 1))
 (segment (start 84.8062 77.5482) (end 84.9022 77.529) (width 0.25) (layer "F.Cu") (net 1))
 (segment (start 87.15 81.275) (end 87.81 81.195) (width 0.25) (layer "F.Cu") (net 1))
 (segment (start 83.3174 79.1902) (end 84.6076 77.7198) (width 0.25) (layer "F.Cu") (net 1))
 (via (at 88.385 81.0618) (size 0.8) (drill 0.4) (layers "F.Cu" "B.Cu") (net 1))
 (segment (start 89.905 85.99) (end 90.63 86.715) (width 0.25) (layer "B.Cu") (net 1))
 (segment (start 88.1583 83.8254) (end 88.1583 84.3224) (width 0.25) (layer "B.Cu") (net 1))
 (segment (start 88.385 81.0618) (end 88.1583 83.8254) (width 0.25) (layer "B.Cu") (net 1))
 (segment (start 88.1583 84.3224) (end 89.655 85.9168) (width 0.25) (layer "B.Cu") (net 1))
 (segment (start 89.7282 85.99) (end 89.78 85.99) (width 0.25) (layer "B.Cu") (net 1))
 (segment (start 89.78 85.99) (end 89.905 85.99) (width 0.25) (layer "B.Cu") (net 1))
 (segment (start 89.655 85.9168) (end 89.7282 85.99) (width 0.25) (layer "B.Cu") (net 1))
 (segment (start 80.75 81.845) (end 81.41 81.925) (width 0.25) (layer "F.Cu") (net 9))
 (segment (start 78.98 78.6551) (end 80.5 81.7718) (width 0.25) (layer "F.Cu") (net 9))
 (segment (start 80.5 81.7718) (end 80.5732 81.845) (width 0.25) (layer "F.Cu") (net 9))
 (segment (start 80.625 81.845) (end 80.75 81.845) (width 0.25) (layer "F.Cu") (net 9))
 (segment (start 80.5732 81.845) (end 80.625 81.845) (width 0.25) (layer "F.Cu") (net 9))
 (segment (start 77.93 76.55) (end 78.98 78.6551) (width 0.25) (layer "F.Cu") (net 9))
 (segment (start 76.12 74.9) (end 77.93 76.55) (width 0.25) (layer "B.Cu") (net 9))
 (segment (start 80.75 82.495) (end 81.41 82.575) (width 0.25) (layer "F.Cu") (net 10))
 (segment (start 80.5 82.4218) (end 80.5732 82.495) (width 0.25) (layer "F.Cu") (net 10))
 (segment (start 80.625 82.495) (end 80.75 82.495) (width 0.25) (layer "F.Cu") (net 10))
 (segment (start 80.5732 82.495) (end 80.625 82.495) (width 0.25) (layer "F.Cu") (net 10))
 (segment (start 77.93 79.09) (end 80.5 82.4218) (width 0.25) (layer "F.Cu") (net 10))
 (segment (start 76.12 76.17) (end 76.82 77.1501) (width 0.25) (layer "B.Cu") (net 10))
 (segment (start 76.82 77.1501) (end 77.93 79.09) (width 0.25) (layer "B.Cu") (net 10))
 (segment (start 80.75 83.145) (end 81.41 83.225) (width 0.25) (layer "F.Cu") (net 11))
 (segment (start 77.93 81.63) (end 80.5732 83.145) (width 0.25) (layer "F.Cu") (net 11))
 (segment (start 80.625 83.145) (end 80.75 83.145) (width 0.25) (layer "F.Cu") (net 11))
 (segment (start 80.5732 83.145) (end 80.625 83.145) (width 0.25) (layer "F.Cu") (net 11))
 (segment (start 76.82 78.4201) (end 76.88 79.5249) (width 0.25) (layer "B.Cu") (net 11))
 (segment (start 76.12 77.44) (end 76.82 78.4201) (width 0.25) (layer "B.Cu") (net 11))
 (segment (start 76.88 79.5249) (end 77.93 81.63) (width 0.25) (layer "B.Cu") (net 11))
 (segment (start 80.75 83.955) (end 81.41 83.875) (width 0.25) (layer "F.Cu") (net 12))
 (segment (start 76.7028 79.28) (end 76.82 79.3972) (width 0.25) (layer "F.Cu") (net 12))
 (segment (start 80.5732 83.955) (end 80.625 83.955) (width 0.25) (layer "F.Cu") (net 12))
 (segment (start 76.82 79.3972) (end 76.88 82.0649) (width 0.25) (layer "F.Cu") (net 12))
 (segment (start 76.12 78.71) (end 76.7028 79.28) (width 0.25) (layer "F.Cu") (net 12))
 (segment (start 76.88 82.0649) (end 77.93 84.17) (width 0.25) (layer "F.Cu") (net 12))
 (segment (start 80.625 83.955) (end 80.75 83.955) (width 0.25) (layer "F.Cu") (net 12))
 (segment (start 77.93 84.17) (end 80.5732 83.955) (width 0.25) (layer "F.Cu") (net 12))
 (segment (start 89.58 78.6601) (end 88.985 81.3103) (width 0.25) (layer "F.Cu") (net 5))
 (segment (start 87.81 81.845) (end 87.15 81.925) (width 0.25) (layer "F.Cu") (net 5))
 (segment (start 87.935 81.845) (end 87.81 81.845) (width 0.25) (layer "F.Cu") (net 5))
 (segment (start 90.63 76.555) (end 89.58 78.6601) (width 0.25) (layer "F.Cu") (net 5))
 (segment (start 88.985 81.3103) (end 88.6335 81.6618) (width 0.25) (layer "F.Cu") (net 5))
 (segment (start 87.9868 81.845) (end 87.935 81.845) (width 0.25) (layer "F.Cu") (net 5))
 (segment (start 88.6335 81.6618) (end 87.9868 81.845) (width 0.25) (layer "F.Cu") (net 5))
 (segment (start 87.9868 82.495) (end 87.935 82.495) (width 0.25) (layer "F.Cu") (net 4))
 (segment (start 90.63 79.095) (end 89.31 81.4449) (width 0.25) (layer "F.Cu") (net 4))
 (segment (start 88.7681 81.9868) (end 87.9868 82.495) (width 0.25) (layer "F.Cu") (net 4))
 (segment (start 87.81 82.495) (end 87.15 82.575) (width 0.25) (layer "F.Cu") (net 4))
 (segment (start 89.31 81.4449) (end 88.7681 81.9868) (width 0.25) (layer "F.Cu") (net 4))
 (segment (start 87.935 82.495) (end 87.81 82.495) (width 0.25) (layer "F.Cu") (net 4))
 (segment (start 87.81 83.145) (end 87.15 83.225) (width 0.25) (layer "F.Cu") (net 3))
 (segment (start 87.9868 83.145) (end 87.935 83.145) (width 0.25) (layer "F.Cu") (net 3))
 (segment (start 90.63 81.635) (end 87.9868 83.145) (width 0.25) (layer "F.Cu") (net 3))
 (segment (start 87.935 83.145) (end 87.81 83.145) (width 0.25) (layer "F.Cu") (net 3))
 (segment (start 90.63 84.175) (end 89.0068 83.4739) (width 0.25) (layer "F.Cu") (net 2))
 (segment (start 89.0068 83.4739) (end 88.5098 83.4739) (width 0.25) (layer "F.Cu") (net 2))
 (segment (start 87.935 83.795) (end 87.81 83.795) (width 0.25) (layer "F.Cu") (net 2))
 (segment (start 88.5098 83.4739) (end 87.9868 83.795) (width 0.25) (layer "F.Cu") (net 2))
 (segment (start 87.9868 83.795) (end 87.935 83.795) (width 0.25) (layer "F.Cu") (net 2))
 (segment (start 87.81 83.795) (end 87.15 83.875) (width 0.25) (layer "F.Cu") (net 2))
 (segment (start 86.365 85.255) (end 86.49 85.255) (width 0.25) (layer "F.Cu") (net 7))
 (segment (start 85.7667 86.0554) (end 85.774 86.0481) (width 0.25) (layer "F.Cu") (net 7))
 (segment (start 90.63 71.475) (end 88.2568 71.73) (width 0.25) (layer "F.Cu") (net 7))
 (segment (start 88.08 71.73) (end 87.455 72.105) (width 0.25) (layer "F.Cu") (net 7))
 (segment (start 79.5022 74.6494) (end 80.4773 75.6245) (width 0.25) (layer "F.Cu") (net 7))
 (segment (start 80.4773 75.6245) (end 80.5706 75.7178) (width 0.25) (layer "F.Cu") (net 7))
 (segment (start 83.3554 76.2455) (end 84.3952 75.8148) (width 0.25) (layer "F.Cu") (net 7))
 (segment (start 83.3216 76.2456) (end 83.3554 76.2455) (width 0.25) (layer "F.Cu") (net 7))
 (segment (start 80.5706 75.7178) (end 80.6144 75.736) (width 0.25) (layer "F.Cu") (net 7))
 (segment (start 90.63 71.475) (end 91.68 73.5801) (width 0.25) (layer "F.Cu") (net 7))
 (segment (start 86.83 72.48) (end 87.455 72.105) (width 0.25) (layer "F.Cu") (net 7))
 (segment (start 86.24 85.3282) (end 86.3132 85.255) (width 0.25) (layer "F.Cu") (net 7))
 (segment (start 84.5982 75.7307) (end 84.6294 75.7177) (width 0.25) (layer "F.Cu") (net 7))
 (segment (start 91.68 73.5801) (end 91.68 83.7401) (width 0.25) (layer "F.Cu") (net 7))
 (segment (start 91.0649 85.225) (end 87.935 85.225) (width 0.25) (layer "F.Cu") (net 7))
 (segment (start 85.774 86.0481) (end 86.24 85.3282) (width 0.25) (layer "F.Cu") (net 7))
 (segment (start 86.58 72.5532) (end 86.6532 72.48) (width 0.25) (layer "F.Cu") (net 7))
 (segment (start 88.205 71.73) (end 88.08 71.73) (width 0.25) (layer "F.Cu") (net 7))
 (segment (start 91.68 83.7401) (end 91.68 84.6099) (width 0.25) (layer "F.Cu") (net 7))
 (segment (start 85.6978 74.6493) (end 86.58 72.5532) (width 0.25) (layer "F.Cu") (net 7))
 (segment (start 87.81 85.225) (end 87.15 85.175) (width 0.25) (layer "F.Cu") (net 7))
 (segment (start 85.28 86.71) (end 85.7667 86.0554) (width 0.25) (layer "F.Cu") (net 7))
 (segment (start 80.6144 75.736) (end 81.8446 76.2456) (width 0.25) (layer "F.Cu") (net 7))
 (segment (start 87.935 85.225) (end 87.81 85.225) (width 0.25) (layer "F.Cu") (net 7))
 (segment (start 88.2568 71.73) (end 88.205 71.73) (width 0.25) (layer "F.Cu") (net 7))
 (segment (start 86.49 85.255) (end 87.15 85.175) (width 0.25) (layer "F.Cu") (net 7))
 (segment (start 81.8446 76.2456) (end 83.1898 76.2456) (width 0.25) (layer "F.Cu") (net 7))
 (segment (start 84.6294 75.7177) (end 85.6045 74.7426) (width 0.25) (layer "F.Cu") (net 7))
 (segment (start 86.705 72.48) (end 86.83 72.48) (width 0.25) (layer "F.Cu") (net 7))
 (segment (start 85.6045 74.7426) (end 85.6978 74.6493) (width 0.25) (layer "F.Cu") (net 7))
 (segment (start 78.98 73.5751) (end 79.5022 74.6494) (width 0.25) (layer "F.Cu") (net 7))
 (segment (start 83.1898 76.2456) (end 83.3216 76.2456) (width 0.25) (layer "F.Cu") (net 7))
 (segment (start 86.6532 72.48) (end 86.705 72.48) (width 0.25) (layer "F.Cu") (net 7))
 (segment (start 84.3952 75.8148) (end 84.5982 75.7307) (width 0.25) (layer "F.Cu") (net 7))
 (segment (start 86.3132 85.255) (end 86.365 85.255) (width 0.25) (layer "F.Cu") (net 7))
 (segment (start 77.93 71.47) (end 78.98 73.5751) (width 0.25) (layer "F.Cu") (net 7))
 (segment (start 91.68 84.6099) (end 91.0649 85.225) (width 0.25) (layer "F.Cu") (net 7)))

